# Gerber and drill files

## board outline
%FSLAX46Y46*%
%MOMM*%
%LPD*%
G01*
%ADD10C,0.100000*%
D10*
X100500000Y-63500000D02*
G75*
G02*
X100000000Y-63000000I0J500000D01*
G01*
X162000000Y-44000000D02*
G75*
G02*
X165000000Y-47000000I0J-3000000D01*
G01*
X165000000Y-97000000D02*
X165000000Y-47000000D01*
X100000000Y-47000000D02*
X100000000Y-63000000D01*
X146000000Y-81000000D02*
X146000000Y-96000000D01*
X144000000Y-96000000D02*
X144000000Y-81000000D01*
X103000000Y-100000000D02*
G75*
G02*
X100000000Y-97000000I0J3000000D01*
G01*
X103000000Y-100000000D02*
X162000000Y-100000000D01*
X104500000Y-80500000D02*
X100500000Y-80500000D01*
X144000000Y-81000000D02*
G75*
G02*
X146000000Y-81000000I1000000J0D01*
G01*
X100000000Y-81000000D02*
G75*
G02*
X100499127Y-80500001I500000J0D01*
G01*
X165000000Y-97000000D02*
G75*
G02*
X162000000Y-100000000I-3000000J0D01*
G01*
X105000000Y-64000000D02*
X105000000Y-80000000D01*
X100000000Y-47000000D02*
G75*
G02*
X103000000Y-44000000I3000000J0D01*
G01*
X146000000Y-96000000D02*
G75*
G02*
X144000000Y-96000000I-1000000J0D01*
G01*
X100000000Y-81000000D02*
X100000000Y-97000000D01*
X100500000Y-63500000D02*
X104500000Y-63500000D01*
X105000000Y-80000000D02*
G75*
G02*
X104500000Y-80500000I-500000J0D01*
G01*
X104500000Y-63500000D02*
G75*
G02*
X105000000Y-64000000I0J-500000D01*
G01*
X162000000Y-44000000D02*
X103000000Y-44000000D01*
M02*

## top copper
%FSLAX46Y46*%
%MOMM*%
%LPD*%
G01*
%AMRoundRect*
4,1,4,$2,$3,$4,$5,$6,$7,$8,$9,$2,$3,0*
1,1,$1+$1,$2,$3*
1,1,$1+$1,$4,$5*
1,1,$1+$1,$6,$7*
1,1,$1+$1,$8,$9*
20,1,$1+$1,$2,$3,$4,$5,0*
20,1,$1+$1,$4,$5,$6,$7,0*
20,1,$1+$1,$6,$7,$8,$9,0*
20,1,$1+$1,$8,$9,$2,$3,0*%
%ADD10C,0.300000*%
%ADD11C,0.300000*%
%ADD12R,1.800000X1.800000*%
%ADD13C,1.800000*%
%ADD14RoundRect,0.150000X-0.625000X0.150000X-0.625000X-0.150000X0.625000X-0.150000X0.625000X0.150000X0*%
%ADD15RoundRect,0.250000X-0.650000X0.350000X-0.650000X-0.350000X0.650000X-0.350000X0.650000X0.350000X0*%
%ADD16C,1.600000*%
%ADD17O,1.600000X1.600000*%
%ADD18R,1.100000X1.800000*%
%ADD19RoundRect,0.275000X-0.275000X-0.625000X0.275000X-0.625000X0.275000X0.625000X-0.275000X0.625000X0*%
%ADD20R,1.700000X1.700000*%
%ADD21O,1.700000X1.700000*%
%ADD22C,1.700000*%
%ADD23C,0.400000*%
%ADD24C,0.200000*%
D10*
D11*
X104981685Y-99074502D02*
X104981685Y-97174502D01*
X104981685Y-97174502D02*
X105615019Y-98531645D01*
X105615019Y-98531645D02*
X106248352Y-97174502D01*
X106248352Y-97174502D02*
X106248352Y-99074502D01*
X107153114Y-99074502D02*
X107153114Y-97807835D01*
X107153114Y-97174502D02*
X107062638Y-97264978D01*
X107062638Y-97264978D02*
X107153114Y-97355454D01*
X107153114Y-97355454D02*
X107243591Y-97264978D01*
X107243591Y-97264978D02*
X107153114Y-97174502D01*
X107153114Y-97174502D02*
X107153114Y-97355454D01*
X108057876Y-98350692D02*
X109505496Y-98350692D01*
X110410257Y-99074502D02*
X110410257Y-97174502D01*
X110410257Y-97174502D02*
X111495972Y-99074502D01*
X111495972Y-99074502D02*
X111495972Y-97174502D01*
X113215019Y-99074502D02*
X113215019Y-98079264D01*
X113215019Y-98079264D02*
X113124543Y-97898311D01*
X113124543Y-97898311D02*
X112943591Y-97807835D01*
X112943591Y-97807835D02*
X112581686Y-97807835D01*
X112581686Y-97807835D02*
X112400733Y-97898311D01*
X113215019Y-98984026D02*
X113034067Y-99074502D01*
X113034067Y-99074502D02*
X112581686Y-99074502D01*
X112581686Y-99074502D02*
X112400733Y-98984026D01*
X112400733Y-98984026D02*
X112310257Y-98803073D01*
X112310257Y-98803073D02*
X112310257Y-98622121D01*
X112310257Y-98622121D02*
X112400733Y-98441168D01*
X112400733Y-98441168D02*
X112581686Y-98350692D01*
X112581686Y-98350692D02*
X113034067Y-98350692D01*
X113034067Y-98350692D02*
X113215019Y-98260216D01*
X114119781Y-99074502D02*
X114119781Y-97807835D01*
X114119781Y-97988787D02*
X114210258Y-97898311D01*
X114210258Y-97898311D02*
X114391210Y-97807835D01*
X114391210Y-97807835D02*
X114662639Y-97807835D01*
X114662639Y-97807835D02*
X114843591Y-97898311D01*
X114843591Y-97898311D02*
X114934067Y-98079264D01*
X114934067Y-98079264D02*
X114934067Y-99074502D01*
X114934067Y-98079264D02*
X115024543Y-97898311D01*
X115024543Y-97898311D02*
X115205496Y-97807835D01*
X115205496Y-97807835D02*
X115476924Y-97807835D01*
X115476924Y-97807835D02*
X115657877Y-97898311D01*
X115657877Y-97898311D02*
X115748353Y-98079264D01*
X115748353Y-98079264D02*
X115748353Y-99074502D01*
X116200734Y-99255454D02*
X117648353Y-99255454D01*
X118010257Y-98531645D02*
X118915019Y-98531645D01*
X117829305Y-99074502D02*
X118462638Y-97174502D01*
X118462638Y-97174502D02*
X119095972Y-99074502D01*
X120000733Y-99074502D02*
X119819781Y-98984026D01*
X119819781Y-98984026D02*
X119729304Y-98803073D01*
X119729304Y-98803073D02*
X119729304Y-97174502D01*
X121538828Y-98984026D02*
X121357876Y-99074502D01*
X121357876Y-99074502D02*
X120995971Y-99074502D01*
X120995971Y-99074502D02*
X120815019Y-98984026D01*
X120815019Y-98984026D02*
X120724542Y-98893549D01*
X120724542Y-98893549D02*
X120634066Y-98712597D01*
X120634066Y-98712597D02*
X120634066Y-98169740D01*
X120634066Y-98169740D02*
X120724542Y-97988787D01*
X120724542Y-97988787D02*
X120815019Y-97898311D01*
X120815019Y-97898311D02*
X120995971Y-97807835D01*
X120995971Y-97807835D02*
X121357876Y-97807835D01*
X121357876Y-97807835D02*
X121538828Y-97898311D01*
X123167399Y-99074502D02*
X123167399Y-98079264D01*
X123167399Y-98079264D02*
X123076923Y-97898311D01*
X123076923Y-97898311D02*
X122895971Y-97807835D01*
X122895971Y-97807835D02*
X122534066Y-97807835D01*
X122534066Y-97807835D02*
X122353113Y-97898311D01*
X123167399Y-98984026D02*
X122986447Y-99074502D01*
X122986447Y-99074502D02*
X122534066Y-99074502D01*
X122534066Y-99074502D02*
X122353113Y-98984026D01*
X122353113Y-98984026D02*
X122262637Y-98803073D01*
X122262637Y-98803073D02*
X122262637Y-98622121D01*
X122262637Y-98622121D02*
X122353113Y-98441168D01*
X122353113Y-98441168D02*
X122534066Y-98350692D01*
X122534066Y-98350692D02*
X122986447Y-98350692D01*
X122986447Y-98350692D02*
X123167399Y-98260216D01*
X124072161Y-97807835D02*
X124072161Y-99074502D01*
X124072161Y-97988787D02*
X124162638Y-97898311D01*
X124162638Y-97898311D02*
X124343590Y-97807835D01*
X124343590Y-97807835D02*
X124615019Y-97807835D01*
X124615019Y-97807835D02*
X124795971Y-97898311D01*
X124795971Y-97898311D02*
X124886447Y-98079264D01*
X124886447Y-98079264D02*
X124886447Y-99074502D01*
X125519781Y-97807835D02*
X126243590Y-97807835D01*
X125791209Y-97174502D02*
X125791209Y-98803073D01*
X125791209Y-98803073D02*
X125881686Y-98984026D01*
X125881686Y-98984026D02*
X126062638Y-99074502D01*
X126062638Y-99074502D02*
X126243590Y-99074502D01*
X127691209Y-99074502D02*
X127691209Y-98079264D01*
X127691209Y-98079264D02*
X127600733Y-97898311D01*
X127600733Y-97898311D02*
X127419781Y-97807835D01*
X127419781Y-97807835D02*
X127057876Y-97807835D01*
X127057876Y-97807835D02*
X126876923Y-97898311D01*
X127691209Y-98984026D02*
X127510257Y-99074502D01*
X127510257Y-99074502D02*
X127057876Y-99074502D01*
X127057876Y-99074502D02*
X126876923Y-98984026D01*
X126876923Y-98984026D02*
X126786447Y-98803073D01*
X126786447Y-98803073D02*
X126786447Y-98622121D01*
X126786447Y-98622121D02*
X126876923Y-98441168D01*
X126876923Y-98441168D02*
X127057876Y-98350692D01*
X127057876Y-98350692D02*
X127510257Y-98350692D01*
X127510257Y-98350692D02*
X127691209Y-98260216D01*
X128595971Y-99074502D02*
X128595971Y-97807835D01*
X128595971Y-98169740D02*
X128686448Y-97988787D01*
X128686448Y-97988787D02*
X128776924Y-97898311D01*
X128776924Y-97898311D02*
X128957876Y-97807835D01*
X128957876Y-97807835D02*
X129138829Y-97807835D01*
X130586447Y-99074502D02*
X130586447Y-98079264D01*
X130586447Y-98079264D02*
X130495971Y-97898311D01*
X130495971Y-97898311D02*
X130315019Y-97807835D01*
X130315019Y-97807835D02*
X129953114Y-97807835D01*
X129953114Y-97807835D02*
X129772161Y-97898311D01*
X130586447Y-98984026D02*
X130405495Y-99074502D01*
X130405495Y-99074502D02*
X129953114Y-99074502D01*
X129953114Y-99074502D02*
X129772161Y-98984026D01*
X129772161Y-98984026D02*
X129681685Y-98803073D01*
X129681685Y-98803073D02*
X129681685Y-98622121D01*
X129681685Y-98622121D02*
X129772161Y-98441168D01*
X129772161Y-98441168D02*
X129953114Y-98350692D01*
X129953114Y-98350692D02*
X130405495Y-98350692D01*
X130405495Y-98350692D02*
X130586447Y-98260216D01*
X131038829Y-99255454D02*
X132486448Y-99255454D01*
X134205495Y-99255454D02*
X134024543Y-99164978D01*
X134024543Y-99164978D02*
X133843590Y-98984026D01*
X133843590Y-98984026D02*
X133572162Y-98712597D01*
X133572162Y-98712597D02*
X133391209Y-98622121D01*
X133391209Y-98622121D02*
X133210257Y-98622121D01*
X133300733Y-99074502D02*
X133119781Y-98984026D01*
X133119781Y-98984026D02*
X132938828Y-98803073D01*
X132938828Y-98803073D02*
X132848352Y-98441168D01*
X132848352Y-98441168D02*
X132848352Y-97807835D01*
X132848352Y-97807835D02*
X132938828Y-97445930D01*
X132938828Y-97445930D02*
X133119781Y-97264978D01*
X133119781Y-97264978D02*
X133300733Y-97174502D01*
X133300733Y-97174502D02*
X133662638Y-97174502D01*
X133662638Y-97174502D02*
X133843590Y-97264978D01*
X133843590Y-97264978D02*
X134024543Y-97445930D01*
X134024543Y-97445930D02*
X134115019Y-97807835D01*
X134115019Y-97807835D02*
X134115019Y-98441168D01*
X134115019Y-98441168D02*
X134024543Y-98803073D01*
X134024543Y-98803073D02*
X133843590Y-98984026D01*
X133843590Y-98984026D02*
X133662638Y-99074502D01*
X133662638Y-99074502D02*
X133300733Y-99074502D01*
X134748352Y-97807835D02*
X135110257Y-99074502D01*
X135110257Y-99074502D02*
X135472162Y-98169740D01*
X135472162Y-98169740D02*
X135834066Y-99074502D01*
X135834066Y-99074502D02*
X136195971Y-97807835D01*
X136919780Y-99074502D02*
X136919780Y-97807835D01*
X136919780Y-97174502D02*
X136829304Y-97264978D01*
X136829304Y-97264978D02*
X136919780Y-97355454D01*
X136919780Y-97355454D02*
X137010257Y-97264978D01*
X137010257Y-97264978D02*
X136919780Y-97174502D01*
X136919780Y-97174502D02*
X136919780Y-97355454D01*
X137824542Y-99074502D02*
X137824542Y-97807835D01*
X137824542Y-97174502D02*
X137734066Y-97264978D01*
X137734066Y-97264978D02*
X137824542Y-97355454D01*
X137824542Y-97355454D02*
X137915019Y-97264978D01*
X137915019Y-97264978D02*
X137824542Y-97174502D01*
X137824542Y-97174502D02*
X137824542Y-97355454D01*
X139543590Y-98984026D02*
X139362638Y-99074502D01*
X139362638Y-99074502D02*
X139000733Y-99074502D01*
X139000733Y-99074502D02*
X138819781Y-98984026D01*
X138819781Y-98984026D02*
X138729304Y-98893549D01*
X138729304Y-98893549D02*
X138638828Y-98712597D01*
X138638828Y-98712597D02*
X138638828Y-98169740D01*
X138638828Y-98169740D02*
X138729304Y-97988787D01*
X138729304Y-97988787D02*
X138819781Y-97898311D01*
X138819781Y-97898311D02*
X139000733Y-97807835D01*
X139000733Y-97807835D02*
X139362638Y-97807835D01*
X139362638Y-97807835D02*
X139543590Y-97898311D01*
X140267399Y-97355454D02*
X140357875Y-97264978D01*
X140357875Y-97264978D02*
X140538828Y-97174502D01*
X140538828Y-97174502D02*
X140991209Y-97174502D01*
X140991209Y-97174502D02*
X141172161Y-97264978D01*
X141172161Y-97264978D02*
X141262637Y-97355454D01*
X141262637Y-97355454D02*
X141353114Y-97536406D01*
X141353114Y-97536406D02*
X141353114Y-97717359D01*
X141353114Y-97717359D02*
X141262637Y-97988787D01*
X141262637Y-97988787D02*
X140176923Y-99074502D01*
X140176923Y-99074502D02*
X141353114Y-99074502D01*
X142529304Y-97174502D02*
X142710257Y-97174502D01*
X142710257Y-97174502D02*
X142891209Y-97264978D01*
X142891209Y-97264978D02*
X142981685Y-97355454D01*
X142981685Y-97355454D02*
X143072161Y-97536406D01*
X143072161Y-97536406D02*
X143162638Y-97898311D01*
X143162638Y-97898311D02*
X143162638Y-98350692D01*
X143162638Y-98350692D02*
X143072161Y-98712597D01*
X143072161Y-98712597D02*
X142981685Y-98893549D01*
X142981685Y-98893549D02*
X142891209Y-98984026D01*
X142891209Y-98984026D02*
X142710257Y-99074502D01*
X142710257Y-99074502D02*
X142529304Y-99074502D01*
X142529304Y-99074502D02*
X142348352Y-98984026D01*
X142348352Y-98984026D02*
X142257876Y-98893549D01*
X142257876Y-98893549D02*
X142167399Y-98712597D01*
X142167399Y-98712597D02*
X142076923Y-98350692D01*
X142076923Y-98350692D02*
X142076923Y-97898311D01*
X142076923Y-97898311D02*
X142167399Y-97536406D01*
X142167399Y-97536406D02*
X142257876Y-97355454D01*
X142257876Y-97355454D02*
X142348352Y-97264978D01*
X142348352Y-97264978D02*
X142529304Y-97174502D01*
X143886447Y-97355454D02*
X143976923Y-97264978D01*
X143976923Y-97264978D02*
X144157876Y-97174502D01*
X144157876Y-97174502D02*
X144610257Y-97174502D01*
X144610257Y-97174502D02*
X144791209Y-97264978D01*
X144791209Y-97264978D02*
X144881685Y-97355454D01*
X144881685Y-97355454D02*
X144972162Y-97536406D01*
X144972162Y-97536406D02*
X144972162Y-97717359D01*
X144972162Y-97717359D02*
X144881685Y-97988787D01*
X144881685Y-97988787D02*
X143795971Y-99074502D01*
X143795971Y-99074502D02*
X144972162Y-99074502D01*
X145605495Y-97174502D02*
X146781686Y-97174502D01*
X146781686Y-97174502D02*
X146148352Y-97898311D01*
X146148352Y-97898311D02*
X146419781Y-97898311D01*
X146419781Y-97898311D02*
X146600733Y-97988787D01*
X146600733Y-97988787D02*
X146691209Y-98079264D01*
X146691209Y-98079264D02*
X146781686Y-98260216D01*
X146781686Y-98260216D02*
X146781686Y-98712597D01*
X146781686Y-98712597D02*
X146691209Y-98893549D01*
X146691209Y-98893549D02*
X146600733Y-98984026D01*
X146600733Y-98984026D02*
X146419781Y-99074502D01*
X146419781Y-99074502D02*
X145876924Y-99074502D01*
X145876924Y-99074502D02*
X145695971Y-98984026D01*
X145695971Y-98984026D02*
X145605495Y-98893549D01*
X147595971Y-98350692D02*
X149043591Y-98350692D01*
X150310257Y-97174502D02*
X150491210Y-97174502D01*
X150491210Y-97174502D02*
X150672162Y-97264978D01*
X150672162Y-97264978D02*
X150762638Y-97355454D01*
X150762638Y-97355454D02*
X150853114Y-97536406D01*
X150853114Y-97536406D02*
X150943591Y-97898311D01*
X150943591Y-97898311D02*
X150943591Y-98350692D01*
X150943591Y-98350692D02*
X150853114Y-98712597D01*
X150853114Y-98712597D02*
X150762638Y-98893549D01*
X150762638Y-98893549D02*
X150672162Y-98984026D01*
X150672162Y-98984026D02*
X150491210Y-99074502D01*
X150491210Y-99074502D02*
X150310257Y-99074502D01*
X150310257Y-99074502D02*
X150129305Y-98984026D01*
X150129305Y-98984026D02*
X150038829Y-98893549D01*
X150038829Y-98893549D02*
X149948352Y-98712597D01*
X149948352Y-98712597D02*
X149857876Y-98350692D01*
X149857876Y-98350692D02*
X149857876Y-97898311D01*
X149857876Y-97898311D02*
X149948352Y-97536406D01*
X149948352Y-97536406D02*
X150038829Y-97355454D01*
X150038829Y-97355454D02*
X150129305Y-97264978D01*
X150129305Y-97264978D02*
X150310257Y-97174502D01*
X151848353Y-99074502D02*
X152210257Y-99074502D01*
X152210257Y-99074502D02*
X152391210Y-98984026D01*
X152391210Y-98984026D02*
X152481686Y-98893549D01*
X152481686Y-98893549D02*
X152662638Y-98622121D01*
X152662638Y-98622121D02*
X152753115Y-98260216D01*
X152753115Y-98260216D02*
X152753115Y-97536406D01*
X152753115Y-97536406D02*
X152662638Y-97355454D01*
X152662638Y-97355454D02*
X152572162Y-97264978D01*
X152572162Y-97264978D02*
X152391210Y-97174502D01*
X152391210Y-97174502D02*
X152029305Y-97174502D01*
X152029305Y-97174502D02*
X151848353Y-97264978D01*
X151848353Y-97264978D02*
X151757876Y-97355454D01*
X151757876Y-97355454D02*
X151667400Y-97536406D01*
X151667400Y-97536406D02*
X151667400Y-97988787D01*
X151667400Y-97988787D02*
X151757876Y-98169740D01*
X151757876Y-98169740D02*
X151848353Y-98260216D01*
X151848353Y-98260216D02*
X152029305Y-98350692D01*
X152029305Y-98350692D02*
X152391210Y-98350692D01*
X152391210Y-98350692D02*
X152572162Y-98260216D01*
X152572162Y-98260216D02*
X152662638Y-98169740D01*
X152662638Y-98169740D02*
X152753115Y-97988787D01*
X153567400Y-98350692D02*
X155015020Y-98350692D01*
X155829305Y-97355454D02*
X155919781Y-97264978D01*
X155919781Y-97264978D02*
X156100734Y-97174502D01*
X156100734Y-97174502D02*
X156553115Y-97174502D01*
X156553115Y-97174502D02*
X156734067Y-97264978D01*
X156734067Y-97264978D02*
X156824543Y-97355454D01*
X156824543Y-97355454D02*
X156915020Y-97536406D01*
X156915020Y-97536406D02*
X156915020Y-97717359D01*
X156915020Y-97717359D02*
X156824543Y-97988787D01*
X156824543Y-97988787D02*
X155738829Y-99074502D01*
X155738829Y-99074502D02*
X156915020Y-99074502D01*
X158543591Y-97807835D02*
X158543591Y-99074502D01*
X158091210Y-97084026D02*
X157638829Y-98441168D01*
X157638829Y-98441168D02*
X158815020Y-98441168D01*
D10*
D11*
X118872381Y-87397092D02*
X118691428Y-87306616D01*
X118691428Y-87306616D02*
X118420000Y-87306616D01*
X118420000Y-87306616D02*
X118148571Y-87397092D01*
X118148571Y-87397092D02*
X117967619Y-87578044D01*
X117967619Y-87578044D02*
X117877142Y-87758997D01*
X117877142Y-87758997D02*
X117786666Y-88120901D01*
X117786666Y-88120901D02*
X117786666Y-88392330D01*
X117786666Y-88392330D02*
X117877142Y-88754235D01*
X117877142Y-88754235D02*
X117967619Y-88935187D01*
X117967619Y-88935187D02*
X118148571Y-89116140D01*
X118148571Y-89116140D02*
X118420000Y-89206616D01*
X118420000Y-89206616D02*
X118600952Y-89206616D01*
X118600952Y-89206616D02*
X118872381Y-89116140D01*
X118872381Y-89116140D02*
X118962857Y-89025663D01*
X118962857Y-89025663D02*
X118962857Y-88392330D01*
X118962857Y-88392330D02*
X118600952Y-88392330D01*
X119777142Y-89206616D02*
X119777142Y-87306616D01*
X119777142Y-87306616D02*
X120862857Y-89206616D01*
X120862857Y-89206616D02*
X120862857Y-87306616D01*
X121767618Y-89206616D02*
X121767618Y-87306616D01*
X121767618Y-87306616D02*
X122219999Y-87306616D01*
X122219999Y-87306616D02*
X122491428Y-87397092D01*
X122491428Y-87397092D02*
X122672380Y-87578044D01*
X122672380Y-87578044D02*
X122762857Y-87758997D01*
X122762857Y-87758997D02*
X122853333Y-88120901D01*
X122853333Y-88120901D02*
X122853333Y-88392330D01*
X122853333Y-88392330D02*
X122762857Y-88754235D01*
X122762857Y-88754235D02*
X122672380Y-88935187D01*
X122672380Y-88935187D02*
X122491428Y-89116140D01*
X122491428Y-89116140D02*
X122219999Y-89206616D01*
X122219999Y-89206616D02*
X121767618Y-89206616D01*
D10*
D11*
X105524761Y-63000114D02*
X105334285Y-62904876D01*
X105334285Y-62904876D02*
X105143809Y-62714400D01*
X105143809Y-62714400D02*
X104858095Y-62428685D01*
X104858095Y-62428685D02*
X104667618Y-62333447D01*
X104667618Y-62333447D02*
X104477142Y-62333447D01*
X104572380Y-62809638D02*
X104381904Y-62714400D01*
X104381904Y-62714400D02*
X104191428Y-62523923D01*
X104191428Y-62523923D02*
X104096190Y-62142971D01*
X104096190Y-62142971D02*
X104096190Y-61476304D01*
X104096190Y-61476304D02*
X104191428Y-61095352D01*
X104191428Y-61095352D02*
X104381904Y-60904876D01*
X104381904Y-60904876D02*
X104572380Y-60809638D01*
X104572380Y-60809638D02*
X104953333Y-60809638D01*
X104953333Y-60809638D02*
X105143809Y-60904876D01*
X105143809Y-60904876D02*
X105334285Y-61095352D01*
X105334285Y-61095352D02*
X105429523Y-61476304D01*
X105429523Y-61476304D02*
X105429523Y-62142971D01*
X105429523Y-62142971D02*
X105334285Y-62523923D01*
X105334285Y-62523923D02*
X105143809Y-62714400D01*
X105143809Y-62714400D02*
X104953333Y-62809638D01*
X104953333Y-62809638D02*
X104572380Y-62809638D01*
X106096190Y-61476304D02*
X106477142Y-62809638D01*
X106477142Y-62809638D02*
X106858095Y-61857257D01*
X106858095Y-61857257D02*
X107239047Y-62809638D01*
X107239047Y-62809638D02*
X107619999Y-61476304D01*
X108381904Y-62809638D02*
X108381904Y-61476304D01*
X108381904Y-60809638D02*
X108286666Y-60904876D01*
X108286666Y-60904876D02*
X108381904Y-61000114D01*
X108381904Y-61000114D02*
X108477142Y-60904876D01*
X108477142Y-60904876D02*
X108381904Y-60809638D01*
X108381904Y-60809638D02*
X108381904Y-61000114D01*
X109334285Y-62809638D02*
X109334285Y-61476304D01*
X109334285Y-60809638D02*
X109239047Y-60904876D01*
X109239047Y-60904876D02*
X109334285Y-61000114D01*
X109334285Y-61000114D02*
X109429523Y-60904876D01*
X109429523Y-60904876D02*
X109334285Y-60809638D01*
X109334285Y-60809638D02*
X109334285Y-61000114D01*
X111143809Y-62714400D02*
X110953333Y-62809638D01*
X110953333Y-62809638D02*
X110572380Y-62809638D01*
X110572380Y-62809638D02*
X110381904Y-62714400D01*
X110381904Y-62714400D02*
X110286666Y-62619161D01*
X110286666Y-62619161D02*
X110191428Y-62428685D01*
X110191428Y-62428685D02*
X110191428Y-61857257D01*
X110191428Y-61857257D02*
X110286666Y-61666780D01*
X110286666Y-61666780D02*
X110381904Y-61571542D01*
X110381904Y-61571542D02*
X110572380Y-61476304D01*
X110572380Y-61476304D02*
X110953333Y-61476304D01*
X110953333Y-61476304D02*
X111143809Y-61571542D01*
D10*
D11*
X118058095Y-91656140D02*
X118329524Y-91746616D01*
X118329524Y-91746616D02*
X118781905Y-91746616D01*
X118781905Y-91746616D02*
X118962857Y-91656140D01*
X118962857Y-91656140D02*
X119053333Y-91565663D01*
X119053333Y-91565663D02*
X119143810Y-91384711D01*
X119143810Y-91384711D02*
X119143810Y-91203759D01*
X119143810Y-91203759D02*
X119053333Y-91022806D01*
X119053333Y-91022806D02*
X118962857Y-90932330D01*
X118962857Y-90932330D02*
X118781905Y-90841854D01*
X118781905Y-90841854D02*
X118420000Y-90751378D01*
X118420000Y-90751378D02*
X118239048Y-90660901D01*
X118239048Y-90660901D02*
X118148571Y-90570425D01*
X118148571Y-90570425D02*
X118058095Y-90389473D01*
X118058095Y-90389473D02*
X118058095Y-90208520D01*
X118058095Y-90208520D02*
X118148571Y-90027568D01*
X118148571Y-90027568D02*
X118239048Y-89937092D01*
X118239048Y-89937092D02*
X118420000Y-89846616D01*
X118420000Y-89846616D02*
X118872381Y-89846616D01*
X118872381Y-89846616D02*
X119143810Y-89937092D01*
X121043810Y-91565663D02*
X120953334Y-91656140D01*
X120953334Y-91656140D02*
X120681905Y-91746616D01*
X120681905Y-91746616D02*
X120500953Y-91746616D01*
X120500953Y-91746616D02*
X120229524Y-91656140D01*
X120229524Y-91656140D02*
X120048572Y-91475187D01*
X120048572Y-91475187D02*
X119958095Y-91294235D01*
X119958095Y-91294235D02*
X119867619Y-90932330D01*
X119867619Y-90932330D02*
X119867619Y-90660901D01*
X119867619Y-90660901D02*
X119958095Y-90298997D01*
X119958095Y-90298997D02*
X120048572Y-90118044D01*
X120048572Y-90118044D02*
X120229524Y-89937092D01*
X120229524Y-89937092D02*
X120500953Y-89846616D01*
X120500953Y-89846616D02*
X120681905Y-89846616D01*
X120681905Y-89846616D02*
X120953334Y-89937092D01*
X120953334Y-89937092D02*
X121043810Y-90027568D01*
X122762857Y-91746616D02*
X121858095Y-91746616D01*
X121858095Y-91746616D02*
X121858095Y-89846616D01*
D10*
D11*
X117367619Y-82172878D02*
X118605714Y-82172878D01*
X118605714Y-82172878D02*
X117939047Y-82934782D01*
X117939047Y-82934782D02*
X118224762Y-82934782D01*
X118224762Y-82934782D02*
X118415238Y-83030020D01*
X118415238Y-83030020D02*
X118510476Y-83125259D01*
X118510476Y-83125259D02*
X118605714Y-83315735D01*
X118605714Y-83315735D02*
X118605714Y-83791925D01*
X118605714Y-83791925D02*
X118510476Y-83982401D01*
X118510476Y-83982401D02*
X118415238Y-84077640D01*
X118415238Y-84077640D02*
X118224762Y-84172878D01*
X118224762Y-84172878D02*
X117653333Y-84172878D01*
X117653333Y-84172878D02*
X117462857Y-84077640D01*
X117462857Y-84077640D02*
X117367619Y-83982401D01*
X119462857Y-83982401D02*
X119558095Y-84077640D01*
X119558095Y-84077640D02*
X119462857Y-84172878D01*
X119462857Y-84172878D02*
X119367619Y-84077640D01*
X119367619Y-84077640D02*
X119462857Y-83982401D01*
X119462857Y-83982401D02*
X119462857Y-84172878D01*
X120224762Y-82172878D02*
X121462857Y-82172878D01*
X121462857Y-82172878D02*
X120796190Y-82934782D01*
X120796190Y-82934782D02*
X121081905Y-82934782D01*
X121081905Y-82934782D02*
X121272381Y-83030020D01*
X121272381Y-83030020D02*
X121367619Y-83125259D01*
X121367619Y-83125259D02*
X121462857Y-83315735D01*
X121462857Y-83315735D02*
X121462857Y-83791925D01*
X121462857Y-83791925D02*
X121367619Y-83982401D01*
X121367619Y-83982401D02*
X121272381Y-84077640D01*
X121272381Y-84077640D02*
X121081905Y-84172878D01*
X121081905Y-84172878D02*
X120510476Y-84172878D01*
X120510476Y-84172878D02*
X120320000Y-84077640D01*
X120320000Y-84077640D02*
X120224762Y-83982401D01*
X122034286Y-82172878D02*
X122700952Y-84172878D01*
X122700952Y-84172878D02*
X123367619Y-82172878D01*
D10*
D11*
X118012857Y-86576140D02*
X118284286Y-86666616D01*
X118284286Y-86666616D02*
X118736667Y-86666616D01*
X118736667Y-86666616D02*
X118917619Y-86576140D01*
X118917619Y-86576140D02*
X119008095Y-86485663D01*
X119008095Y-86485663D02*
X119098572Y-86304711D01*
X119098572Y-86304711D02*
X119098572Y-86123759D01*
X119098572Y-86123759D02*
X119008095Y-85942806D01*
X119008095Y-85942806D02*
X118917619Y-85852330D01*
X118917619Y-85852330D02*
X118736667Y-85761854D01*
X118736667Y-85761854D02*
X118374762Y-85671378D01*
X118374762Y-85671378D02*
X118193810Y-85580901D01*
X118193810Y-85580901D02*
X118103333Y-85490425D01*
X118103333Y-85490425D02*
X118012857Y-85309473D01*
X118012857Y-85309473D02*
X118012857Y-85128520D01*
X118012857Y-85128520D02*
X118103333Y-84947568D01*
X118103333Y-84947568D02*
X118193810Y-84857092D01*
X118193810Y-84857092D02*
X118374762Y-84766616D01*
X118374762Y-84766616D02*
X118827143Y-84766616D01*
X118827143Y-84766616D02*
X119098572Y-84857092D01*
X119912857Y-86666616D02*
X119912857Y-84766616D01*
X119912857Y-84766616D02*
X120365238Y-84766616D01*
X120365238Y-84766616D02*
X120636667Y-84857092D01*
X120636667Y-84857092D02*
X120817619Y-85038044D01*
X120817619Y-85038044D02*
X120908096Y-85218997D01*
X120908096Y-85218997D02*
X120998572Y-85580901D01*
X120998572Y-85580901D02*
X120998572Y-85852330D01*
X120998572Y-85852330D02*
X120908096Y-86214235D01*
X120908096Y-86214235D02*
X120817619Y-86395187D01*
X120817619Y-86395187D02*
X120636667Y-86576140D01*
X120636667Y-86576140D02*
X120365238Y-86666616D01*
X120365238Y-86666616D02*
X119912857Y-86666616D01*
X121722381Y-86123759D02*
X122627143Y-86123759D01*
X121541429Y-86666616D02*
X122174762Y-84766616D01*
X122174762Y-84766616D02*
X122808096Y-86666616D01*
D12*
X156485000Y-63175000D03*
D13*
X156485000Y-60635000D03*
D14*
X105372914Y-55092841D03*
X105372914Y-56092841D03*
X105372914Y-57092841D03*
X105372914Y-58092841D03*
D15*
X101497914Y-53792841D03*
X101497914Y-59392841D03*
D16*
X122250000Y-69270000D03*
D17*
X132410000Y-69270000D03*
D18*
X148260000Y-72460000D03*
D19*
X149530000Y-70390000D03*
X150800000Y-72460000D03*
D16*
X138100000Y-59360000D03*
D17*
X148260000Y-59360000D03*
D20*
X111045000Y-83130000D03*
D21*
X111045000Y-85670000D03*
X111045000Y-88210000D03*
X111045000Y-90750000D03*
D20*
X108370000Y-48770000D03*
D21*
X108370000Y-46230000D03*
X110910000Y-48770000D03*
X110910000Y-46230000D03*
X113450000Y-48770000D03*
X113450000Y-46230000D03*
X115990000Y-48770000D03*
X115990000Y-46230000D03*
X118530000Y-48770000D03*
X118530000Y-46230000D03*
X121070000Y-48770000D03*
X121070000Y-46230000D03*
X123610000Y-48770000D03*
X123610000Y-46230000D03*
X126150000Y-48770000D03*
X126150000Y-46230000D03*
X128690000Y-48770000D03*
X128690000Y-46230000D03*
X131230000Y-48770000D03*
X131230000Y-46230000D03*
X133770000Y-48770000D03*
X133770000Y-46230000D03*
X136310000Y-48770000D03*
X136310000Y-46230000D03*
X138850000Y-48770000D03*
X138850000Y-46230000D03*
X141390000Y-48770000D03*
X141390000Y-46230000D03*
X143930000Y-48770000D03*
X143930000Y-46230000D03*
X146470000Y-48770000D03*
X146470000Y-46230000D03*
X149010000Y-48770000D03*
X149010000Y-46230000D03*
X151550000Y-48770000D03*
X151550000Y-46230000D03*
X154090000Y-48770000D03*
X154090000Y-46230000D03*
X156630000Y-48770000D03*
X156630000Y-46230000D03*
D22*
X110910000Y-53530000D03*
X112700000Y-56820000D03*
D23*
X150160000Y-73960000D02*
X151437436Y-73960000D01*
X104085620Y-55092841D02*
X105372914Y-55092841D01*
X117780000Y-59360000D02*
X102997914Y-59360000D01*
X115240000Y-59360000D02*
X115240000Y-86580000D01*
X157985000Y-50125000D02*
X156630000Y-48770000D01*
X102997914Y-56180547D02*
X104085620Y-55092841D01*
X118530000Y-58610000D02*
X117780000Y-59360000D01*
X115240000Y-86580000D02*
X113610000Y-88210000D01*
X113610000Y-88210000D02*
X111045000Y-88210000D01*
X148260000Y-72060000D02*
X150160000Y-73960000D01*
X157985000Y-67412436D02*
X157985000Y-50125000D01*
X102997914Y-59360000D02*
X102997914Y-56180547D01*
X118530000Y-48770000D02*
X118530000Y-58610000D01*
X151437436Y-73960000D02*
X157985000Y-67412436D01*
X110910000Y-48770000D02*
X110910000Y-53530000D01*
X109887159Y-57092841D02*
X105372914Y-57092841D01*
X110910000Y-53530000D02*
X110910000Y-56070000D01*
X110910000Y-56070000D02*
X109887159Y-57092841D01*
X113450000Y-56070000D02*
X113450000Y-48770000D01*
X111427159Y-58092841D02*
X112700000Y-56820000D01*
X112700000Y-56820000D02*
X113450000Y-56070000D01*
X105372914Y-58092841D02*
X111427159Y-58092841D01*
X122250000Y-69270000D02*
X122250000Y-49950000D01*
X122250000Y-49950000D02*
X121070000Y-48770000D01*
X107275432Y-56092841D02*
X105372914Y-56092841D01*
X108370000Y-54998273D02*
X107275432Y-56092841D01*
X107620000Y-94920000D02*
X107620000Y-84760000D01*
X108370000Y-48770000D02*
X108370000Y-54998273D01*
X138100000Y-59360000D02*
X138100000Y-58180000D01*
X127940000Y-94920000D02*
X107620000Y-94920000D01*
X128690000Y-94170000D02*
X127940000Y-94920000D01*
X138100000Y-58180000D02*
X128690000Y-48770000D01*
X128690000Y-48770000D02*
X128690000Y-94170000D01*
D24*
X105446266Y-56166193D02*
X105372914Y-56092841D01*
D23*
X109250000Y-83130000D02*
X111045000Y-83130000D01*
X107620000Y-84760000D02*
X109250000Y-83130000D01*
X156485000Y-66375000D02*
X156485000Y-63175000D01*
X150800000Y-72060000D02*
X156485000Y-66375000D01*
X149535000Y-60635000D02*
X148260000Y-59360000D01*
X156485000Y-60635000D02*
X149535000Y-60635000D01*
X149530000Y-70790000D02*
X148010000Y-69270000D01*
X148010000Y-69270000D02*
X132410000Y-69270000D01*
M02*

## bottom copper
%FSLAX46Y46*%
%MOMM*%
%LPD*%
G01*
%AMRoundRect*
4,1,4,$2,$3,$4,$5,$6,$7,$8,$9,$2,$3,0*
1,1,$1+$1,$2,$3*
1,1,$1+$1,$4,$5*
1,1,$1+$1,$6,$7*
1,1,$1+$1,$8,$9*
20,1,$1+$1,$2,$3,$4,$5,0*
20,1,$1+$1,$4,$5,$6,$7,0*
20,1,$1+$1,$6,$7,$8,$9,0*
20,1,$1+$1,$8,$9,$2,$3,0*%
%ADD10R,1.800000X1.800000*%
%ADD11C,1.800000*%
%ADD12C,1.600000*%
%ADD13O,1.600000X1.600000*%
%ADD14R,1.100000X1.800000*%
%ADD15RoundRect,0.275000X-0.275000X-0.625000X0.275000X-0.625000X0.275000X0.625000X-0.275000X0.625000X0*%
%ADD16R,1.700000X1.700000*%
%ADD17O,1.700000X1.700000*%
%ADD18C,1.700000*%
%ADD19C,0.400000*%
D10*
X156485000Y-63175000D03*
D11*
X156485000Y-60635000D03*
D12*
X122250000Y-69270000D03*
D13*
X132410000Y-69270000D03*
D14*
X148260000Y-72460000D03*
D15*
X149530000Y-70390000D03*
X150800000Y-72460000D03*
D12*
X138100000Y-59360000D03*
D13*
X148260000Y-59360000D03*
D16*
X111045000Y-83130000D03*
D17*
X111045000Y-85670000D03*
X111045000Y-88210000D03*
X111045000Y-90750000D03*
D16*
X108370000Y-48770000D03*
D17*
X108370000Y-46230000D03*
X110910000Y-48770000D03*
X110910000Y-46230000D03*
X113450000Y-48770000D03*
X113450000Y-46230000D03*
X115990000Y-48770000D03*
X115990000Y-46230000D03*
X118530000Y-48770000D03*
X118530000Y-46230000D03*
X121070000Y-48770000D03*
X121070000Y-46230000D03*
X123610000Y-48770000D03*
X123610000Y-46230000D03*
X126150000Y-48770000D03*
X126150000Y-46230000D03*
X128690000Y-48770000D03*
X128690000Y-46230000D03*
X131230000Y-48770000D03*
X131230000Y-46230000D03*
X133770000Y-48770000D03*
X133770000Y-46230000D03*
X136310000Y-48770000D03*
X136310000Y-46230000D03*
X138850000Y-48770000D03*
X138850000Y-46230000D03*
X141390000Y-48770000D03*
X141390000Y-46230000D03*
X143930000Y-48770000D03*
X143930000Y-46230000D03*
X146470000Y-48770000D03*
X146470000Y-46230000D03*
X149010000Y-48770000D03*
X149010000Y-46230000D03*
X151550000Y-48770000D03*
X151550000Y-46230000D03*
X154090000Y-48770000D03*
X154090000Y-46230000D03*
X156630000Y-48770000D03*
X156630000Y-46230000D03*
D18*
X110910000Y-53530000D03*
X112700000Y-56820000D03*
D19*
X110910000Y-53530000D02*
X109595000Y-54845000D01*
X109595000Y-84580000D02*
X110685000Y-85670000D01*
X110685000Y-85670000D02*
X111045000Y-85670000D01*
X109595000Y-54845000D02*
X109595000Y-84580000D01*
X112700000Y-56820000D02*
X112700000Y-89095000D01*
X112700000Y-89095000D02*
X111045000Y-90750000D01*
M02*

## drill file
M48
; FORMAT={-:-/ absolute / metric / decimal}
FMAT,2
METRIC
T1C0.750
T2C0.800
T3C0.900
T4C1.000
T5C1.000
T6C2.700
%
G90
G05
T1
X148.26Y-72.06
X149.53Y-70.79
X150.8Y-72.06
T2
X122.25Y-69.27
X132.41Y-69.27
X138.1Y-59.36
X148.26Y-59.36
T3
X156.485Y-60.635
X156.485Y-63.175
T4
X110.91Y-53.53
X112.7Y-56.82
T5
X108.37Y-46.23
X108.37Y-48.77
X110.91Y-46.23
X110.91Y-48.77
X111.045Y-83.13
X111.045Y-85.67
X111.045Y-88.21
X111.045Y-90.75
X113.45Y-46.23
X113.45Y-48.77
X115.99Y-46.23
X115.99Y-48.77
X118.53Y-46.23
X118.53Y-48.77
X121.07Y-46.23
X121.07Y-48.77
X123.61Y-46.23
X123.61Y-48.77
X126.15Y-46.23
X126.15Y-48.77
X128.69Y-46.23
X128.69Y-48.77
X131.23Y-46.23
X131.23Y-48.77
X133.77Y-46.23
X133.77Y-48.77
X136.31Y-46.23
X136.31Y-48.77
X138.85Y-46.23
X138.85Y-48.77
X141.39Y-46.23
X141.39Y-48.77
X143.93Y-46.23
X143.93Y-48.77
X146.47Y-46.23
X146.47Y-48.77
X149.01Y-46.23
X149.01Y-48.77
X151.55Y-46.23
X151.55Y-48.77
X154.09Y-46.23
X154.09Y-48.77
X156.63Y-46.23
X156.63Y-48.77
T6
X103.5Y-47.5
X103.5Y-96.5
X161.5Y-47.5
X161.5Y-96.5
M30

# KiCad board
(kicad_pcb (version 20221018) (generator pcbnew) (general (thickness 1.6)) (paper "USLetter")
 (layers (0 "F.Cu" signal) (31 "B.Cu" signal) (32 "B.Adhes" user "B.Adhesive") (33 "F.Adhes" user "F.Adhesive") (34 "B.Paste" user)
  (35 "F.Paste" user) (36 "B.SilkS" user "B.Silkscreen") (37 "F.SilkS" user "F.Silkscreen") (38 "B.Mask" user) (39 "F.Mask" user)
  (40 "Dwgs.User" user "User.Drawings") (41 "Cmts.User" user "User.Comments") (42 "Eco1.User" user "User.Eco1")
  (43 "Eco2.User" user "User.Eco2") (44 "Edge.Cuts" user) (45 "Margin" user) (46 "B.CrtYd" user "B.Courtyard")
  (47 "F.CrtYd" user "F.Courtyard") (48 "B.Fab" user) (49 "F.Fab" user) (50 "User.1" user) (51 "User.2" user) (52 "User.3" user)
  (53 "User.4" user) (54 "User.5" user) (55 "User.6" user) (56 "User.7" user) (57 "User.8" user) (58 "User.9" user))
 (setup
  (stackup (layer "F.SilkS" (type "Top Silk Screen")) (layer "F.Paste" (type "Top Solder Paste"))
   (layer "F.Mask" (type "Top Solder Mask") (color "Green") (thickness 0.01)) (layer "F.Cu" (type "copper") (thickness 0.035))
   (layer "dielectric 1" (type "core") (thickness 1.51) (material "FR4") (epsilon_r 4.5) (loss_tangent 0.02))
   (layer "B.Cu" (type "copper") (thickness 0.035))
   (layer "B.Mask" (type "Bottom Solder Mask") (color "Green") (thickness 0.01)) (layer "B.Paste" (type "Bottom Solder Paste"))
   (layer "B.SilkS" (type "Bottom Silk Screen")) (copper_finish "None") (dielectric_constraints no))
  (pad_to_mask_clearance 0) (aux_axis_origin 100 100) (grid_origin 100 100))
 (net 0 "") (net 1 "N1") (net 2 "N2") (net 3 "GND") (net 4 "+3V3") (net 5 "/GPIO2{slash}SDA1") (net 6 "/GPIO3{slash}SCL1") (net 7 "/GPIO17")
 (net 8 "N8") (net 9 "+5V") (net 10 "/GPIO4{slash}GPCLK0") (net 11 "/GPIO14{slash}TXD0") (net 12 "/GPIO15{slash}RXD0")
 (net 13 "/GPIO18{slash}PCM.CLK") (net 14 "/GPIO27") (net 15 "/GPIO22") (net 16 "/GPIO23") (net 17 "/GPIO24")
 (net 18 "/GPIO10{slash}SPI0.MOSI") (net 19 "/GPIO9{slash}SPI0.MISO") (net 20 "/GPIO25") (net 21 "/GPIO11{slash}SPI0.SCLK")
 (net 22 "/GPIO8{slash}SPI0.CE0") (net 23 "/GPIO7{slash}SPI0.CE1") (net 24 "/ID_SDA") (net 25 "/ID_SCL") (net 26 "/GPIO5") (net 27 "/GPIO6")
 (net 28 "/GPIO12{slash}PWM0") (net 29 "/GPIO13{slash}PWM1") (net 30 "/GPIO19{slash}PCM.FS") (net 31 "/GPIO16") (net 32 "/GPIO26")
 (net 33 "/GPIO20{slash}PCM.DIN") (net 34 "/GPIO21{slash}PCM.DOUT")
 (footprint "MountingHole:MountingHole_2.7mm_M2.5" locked (layer "F.Cu") (at 161.5 47.5)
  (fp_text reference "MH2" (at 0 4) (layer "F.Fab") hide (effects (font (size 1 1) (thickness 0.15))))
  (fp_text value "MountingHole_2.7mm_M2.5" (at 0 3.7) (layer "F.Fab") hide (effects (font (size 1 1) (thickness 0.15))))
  (pad "" np_thru_hole circle locked (at 0 0) (size 2.7 2.7) (drill 2.7) (layers "*.Cu" "*.Mask")))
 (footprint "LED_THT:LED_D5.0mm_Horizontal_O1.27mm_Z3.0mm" (layer "F.Cu") (at 156.485 63.175 90)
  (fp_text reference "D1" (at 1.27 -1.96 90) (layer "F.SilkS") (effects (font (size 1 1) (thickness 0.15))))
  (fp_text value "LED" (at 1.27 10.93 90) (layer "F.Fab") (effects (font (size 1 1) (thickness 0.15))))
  (pad "1" thru_hole rect (at 0 0 90) (size 1.8 1.8) (drill 0.9) (layers "*.Cu" "*.Mask") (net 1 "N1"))
  (pad "2" thru_hole circle (at 2.54 0 90) (size 1.8 1.8) (drill 0.9) (layers "*.Cu" "*.Mask") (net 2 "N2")))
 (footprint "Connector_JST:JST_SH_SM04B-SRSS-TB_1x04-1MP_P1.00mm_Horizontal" (layer "F.Cu") (at 103.372914 56.592841 -90)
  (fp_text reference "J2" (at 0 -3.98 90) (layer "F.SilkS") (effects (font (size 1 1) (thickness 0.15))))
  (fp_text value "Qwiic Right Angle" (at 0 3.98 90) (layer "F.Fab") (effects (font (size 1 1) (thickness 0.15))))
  (pad "1" smd roundrect (at -1.5 -2 270) (size 0.6 1.55) (layers "F.Cu" "F.Paste" "F.Mask") (roundrect_rratio 0.25) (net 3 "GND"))
  (pad "2" smd roundrect (at -0.5 -2 270) (size 0.6 1.55) (layers "F.Cu" "F.Paste" "F.Mask") (roundrect_rratio 0.25) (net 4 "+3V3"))
  (pad "3" smd roundrect (at 0.5 -2 270) (size 0.6 1.55) (layers "F.Cu" "F.Paste" "F.Mask") (roundrect_rratio 0.25)
   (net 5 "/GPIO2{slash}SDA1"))
  (pad "4" smd roundrect (at 1.5 -2 270) (size 0.6 1.55) (layers "F.Cu" "F.Paste" "F.Mask") (roundrect_rratio 0.25)
   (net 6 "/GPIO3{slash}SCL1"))
  (pad "MP" smd roundrect (at -2.8 1.875 270) (size 1.2 1.8) (layers "F.Cu" "F.Paste" "F.Mask") (roundrect_rratio 0.2083333333))
  (pad "MP" smd roundrect (at 2.8 1.875 270) (size 1.2 1.8) (layers "F.Cu" "F.Paste" "F.Mask") (roundrect_rratio 0.2083333333)))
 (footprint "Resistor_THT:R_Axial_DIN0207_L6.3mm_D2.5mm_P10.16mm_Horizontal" (layer "F.Cu") (at 122.25 69.27)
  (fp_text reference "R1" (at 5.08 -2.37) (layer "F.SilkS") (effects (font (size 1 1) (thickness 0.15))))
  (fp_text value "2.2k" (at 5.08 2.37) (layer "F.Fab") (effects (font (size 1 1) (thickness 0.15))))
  (pad "1" thru_hole circle (at 0 0) (size 1.6 1.6) (drill 0.8) (layers "*.Cu" "*.Mask") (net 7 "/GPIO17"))
  (pad "2" thru_hole oval (at 10.16 0) (size 1.6 1.6) (drill 0.8) (layers "*.Cu" "*.Mask") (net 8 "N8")))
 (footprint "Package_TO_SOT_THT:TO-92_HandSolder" (layer "F.Cu") (at 148.26 72.06)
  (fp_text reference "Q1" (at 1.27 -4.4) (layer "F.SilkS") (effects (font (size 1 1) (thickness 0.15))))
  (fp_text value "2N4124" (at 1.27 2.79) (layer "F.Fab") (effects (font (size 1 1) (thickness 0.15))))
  (pad "1" thru_hole rect (at 0 0) (size 1.1 1.8) (drill 0.75 (offset 0 0.4)) (layers "*.Cu" "*.Mask") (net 3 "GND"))
  (pad "2" thru_hole roundrect (at 1.27 -1.27) (size 1.1 1.8) (drill 0.75 (offset 0 -0.4)) (layers "*.Cu" "*.Mask") (roundrect_rratio 0.25)
   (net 8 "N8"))
  (pad "3" thru_hole roundrect (at 2.54 0) (size 1.1 1.8) (drill 0.75 (offset 0 0.4)) (layers "*.Cu" "*.Mask") (roundrect_rratio 0.25)
   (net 1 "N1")))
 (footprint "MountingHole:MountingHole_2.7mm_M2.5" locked (layer "F.Cu") (at 103.5 96.5)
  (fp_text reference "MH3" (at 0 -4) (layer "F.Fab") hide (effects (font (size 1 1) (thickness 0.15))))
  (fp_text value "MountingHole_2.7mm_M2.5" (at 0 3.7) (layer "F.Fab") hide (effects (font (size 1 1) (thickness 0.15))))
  (pad "" np_thru_hole circle locked (at 0 0) (size 2.7 2.7) (drill 2.7) (layers "*.Cu" "*.Mask")))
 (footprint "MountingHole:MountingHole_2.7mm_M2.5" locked (layer "F.Cu") (at 103.5 47.5)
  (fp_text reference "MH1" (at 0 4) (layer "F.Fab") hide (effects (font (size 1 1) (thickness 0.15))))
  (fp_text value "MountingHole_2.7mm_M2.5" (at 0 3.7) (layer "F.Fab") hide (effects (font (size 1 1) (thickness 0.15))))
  (pad "" np_thru_hole circle locked (at 0 0) (size 2.7 2.7) (drill 2.7) (layers "*.Cu" "*.Mask")))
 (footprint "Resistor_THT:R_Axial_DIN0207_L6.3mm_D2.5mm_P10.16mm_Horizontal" (layer "F.Cu") (at 138.1 59.36)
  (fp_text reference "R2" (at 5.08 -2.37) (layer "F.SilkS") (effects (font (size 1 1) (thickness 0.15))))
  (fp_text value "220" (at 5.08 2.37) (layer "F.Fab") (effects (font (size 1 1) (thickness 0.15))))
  (pad "1" thru_hole circle (at 0 0) (size 1.6 1.6) (drill 0.8) (layers "*.Cu" "*.Mask") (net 4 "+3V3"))
  (pad "2" thru_hole oval (at 10.16 0) (size 1.6 1.6) (drill 0.8) (layers "*.Cu" "*.Mask") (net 2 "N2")))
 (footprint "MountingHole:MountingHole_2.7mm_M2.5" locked (layer "F.Cu") (at 161.5 96.5)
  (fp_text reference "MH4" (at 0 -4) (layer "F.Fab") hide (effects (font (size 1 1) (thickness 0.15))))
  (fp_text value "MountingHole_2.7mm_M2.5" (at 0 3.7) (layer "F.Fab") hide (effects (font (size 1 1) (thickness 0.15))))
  (pad "" np_thru_hole circle locked (at 0 0) (size 2.7 2.7) (drill 2.7) (layers "*.Cu" "*.Mask")))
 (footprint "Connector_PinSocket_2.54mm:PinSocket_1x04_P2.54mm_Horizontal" (layer "F.Cu") (at 111.045 83.13)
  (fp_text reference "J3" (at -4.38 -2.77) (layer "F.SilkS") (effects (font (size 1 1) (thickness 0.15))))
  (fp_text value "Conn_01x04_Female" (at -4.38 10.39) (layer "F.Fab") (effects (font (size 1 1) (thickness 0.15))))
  (pad "1" thru_hole rect (at 0 0) (size 1.7 1.7) (drill 1) (layers "*.Cu" "*.Mask") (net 4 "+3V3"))
  (pad "2" thru_hole oval (at 0 2.54) (size 1.7 1.7) (drill 1) (layers "*.Cu" "*.Mask") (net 5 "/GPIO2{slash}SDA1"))
  (pad "3" thru_hole oval (at 0 5.08) (size 1.7 1.7) (drill 1) (layers "*.Cu" "*.Mask") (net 3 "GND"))
  (pad "4" thru_hole oval (at 0 7.62) (size 1.7 1.7) (drill 1) (layers "*.Cu" "*.Mask") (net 6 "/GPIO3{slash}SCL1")))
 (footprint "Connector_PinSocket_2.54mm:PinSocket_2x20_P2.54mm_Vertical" (layer "B.Cu") (at 108.37 48.77 -90)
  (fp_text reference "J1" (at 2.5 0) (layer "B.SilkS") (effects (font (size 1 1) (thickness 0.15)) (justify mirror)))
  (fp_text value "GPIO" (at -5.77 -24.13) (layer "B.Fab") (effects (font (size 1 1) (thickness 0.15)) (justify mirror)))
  (pad "1" thru_hole rect (at 0 0 270) (size 1.7 1.7) (drill 1) (layers "*.Cu" "*.Mask") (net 4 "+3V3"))
  (pad "2" thru_hole oval (at -2.54 0 270) (size 1.7 1.7) (drill 1) (layers "*.Cu" "*.Mask") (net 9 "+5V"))
  (pad "3" thru_hole oval (at 0 -2.54 270) (size 1.7 1.7) (drill 1) (layers "*.Cu" "*.Mask") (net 5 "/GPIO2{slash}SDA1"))
  (pad "4" thru_hole oval (at -2.54 -2.54 270) (size 1.7 1.7) (drill 1) (layers "*.Cu" "*.Mask") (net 9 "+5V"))
  (pad "5" thru_hole oval (at 0 -5.08 270) (size 1.7 1.7) (drill 1) (layers "*.Cu" "*.Mask") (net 6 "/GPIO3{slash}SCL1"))
  (pad "6" thru_hole oval (at -2.54 -5.08 270) (size 1.7 1.7) (drill 1) (layers "*.Cu" "*.Mask") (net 3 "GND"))
  (pad "7" thru_hole oval (at 0 -7.62 270) (size 1.7 1.7) (drill 1) (layers "*.Cu" "*.Mask") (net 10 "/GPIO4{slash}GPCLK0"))
  (pad "8" thru_hole oval (at -2.54 -7.62 270) (size 1.7 1.7) (drill 1) (layers "*.Cu" "*.Mask") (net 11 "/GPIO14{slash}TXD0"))
  (pad "9" thru_hole oval (at 0 -10.16 270) (size 1.7 1.7) (drill 1) (layers "*.Cu" "*.Mask") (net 3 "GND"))
  (pad "10" thru_hole oval (at -2.54 -10.16 270) (size 1.7 1.7) (drill 1) (layers "*.Cu" "*.Mask") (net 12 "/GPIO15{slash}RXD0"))
  (pad "11" thru_hole oval (at 0 -12.7 270) (size 1.7 1.7) (drill 1) (layers "*.Cu" "*.Mask") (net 7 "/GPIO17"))
  (pad "12" thru_hole oval (at -2.54 -12.7 270) (size 1.7 1.7) (drill 1) (layers "*.Cu" "*.Mask") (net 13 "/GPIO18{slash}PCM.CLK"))
  (pad "13" thru_hole oval (at 0 -15.24 270) (size 1.7 1.7) (drill 1) (layers "*.Cu" "*.Mask") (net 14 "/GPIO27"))
  (pad "14" thru_hole oval (at -2.54 -15.24 270) (size 1.7 1.7) (drill 1) (layers "*.Cu" "*.Mask") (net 3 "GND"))
  (pad "15" thru_hole oval (at 0 -17.78 270) (size 1.7 1.7) (drill 1) (layers "*.Cu" "*.Mask") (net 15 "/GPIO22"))
  (pad "16" thru_hole oval (at -2.54 -17.78 270) (size 1.7 1.7) (drill 1) (layers "*.Cu" "*.Mask") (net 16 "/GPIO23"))
  (pad "17" thru_hole oval (at 0 -20.32 270) (size 1.7 1.7) (drill 1) (layers "*.Cu" "*.Mask") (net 4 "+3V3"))
  (pad "18" thru_hole oval (at -2.54 -20.32 270) (size 1.7 1.7) (drill 1) (layers "*.Cu" "*.Mask") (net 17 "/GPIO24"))
  (pad "19" thru_hole oval (at 0 -22.86 270) (size 1.7 1.7) (drill 1) (layers "*.Cu" "*.Mask") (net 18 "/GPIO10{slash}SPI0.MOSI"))
  (pad "20" thru_hole oval (at -2.54 -22.86 270) (size 1.7 1.7) (drill 1) (layers "*.Cu" "*.Mask") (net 3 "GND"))
  (pad "21" thru_hole oval (at 0 -25.4 270) (size 1.7 1.7) (drill 1) (layers "*.Cu" "*.Mask") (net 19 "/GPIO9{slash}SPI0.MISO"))
  (pad "22" thru_hole oval (at -2.54 -25.4 270) (size 1.7 1.7) (drill 1) (layers "*.Cu" "*.Mask") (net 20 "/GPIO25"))
  (pad "23" thru_hole oval (at 0 -27.94 270) (size 1.7 1.7) (drill 1) (layers "*.Cu" "*.Mask") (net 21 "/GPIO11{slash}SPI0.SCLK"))
  (pad "24" thru_hole oval (at -2.54 -27.94 270) (size 1.7 1.7) (drill 1) (layers "*.Cu" "*.Mask") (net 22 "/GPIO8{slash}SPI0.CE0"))
  (pad "25" thru_hole oval (at 0 -30.48 270) (size 1.7 1.7) (drill 1) (layers "*.Cu" "*.Mask") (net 3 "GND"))
  (pad "26" thru_hole oval (at -2.54 -30.48 270) (size 1.7 1.7) (drill 1) (layers "*.Cu" "*.Mask") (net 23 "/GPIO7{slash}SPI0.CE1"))
  (pad "27" thru_hole oval (at 0 -33.02 270) (size 1.7 1.7) (drill 1) (layers "*.Cu" "*.Mask") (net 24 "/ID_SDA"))
  (pad "28" thru_hole oval (at -2.54 -33.02 270) (size 1.7 1.7) (drill 1) (layers "*.Cu" "*.Mask") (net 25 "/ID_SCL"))
  (pad "29" thru_hole oval (at 0 -35.56 270) (size 1.7 1.7) (drill 1) (layers "*.Cu" "*.Mask") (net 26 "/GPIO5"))
  (pad "30" thru_hole oval (at -2.54 -35.56 270) (size 1.7 1.7) (drill 1) (layers "*.Cu" "*.Mask") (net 3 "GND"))
  (pad "31" thru_hole oval (at 0 -38.1 270) (size 1.7 1.7) (drill 1) (layers "*.Cu" "*.Mask") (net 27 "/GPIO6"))
  (pad "32" thru_hole oval (at -2.54 -38.1 270) (size 1.7 1.7) (drill 1) (layers "*.Cu" "*.Mask") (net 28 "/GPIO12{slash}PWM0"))
  (pad "33" thru_hole oval (at 0 -40.64 270) (size 1.7 1.7) (drill 1) (layers "*.Cu" "*.Mask") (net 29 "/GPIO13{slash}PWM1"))
  (pad "34" thru_hole oval (at -2.54 -40.64 270) (size 1.7 1.7) (drill 1) (layers "*.Cu" "*.Mask") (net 3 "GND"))
  (pad "35" thru_hole oval (at 0 -43.18 270) (size 1.7 1.7) (drill 1) (layers "*.Cu" "*.Mask") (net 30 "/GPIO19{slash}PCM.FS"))
  (pad "36" thru_hole oval (at -2.54 -43.18 270) (size 1.7 1.7) (drill 1) (layers "*.Cu" "*.Mask") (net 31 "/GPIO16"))
  (pad "37" thru_hole oval (at 0 -45.72 270) (size 1.7 1.7) (drill 1) (layers "*.Cu" "*.Mask") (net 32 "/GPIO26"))
  (pad "38" thru_hole oval (at -2.54 -45.72 270) (size 1.7 1.7) (drill 1) (layers "*.Cu" "*.Mask") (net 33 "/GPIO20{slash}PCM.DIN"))
  (pad "39" thru_hole oval (at 0 -48.26 270) (size 1.7 1.7) (drill 1) (layers "*.Cu" "*.Mask") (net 3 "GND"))
  (pad "40" thru_hole oval (at -2.54 -48.26 270) (size 1.7 1.7) (drill 1) (layers "*.Cu" "*.Mask") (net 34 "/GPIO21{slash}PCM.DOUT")))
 (gr_arc (start 100.5 63.5) (mid 100.146447 63.353553) (end 100 63) (stroke (width 0.1) (type solid)) (layer "Edge.Cuts"))
 (gr_arc (start 162 44) (mid 164.12132 44.87868) (end 165 47) (stroke (width 0.1) (type solid)) (layer "Edge.Cuts"))
 (gr_line (start 165 97) (end 165 47) (stroke (width 0.1) (type solid)) (layer "Edge.Cuts"))
 (gr_line (start 100 47) (end 100 63) (stroke (width 0.1) (type solid)) (layer "Edge.Cuts"))
 (gr_line (start 146 81) (end 146 96) (stroke (width 0.1) (type solid)) (layer "Edge.Cuts"))
 (gr_line (start 144 96) (end 144 81) (stroke (width 0.1) (type solid)) (layer "Edge.Cuts"))
 (gr_arc (start 103 100) (mid 100.87868 99.12132) (end 100 97) (stroke (width 0.1) (type solid)) (layer "Edge.Cuts"))
 (gr_line (start 103 100) (end 162 100) (stroke (width 0.1) (type solid)) (layer "Edge.Cuts"))
 (gr_line (start 104.5 80.5) (end 100.5 80.5) (stroke (width 0.1) (type solid)) (layer "Edge.Cuts"))
 (gr_arc (start 144 81) (mid 145 80) (end 146 81) (stroke (width 0.1) (type solid)) (layer "Edge.Cuts"))
 (gr_arc (start 100 81) (mid 100.146138 80.646755) (end 100.499127 80.500001) (stroke (width 0.1) (type solid)) (layer "Edge.Cuts"))
 (gr_arc (start 165 97) (mid 164.12132 99.12132) (end 162 100) (stroke (width 0.1) (type solid)) (layer "Edge.Cuts"))
 (gr_line (start 105 64) (end 105 80) (stroke (width 0.1) (type solid)) (layer "Edge.Cuts"))
 (gr_arc (start 100 47) (mid 100.87868 44.87868) (end 103 44) (stroke (width 0.1) (type solid)) (layer "Edge.Cuts"))
 (gr_arc (start 146 96) (mid 145 97) (end 144 96) (stroke (width 0.1) (type solid)) (layer "Edge.Cuts"))
 (gr_line (start 100 81) (end 100 97) (stroke (width 0.1) (type solid)) (layer "Edge.Cuts"))
 (gr_line (start 100.5 63.5) (end 104.5 63.5) (stroke (width 0.1) (type solid)) (layer "Edge.Cuts"))
 (gr_arc (start 105 80) (mid 104.853553 80.353553) (end 104.5 80.5) (stroke (width 0.1) (type solid)) (layer "Edge.Cuts"))
 (gr_arc (start 104.5 63.5) (mid 104.853553 63.646447) (end 105 64) (stroke (width 0.1) (type solid)) (layer "Edge.Cuts"))
 (gr_line (start 162 44) (end 103 44) (stroke (width 0.1) (type solid)) (layer "Edge.Cuts"))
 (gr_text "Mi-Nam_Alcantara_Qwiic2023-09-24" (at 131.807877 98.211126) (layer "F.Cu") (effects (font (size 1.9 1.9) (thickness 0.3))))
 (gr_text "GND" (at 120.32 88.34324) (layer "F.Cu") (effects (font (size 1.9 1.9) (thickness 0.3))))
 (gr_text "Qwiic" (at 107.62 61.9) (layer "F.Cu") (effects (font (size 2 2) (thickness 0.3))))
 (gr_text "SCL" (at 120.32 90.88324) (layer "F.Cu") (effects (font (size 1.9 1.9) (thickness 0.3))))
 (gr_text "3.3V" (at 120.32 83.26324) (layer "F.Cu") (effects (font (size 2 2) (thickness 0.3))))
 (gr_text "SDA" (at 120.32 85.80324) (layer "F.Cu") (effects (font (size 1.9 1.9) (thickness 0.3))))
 (segment (start 150.16 73.96) (end 151.437436 73.96) (width 0.4) (layer "F.Cu") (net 3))
 (segment (start 104.08562 55.092841) (end 105.372914 55.092841) (width 0.4) (layer "F.Cu") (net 3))
 (segment (start 117.78 59.36) (end 102.997914 59.36) (width 0.4) (layer "F.Cu") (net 3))
 (segment (start 115.24 59.36) (end 115.24 86.58) (width 0.4) (layer "F.Cu") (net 3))
 (segment (start 157.985 50.125) (end 156.63 48.77) (width 0.4) (layer "F.Cu") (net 3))
 (segment (start 102.997914 56.180547) (end 104.08562 55.092841) (width 0.4) (layer "F.Cu") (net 3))
 (segment (start 118.53 58.61) (end 117.78 59.36) (width 0.4) (layer "F.Cu") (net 3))
 (segment (start 115.24 86.58) (end 113.61 88.21) (width 0.4) (layer "F.Cu") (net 3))
 (segment (start 113.61 88.21) (end 111.045 88.21) (width 0.4) (layer "F.Cu") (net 3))
 (segment (start 148.26 72.06) (end 150.16 73.96) (width 0.4) (layer "F.Cu") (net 3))
 (segment (start 157.985 67.412436) (end 157.985 50.125) (width 0.4) (layer "F.Cu") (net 3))
 (segment (start 102.997914 59.36) (end 102.997914 56.180547) (width 0.4) (layer "F.Cu") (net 3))
 (segment (start 118.53 48.77) (end 118.53 58.61) (width 0.4) (layer "F.Cu") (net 3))
 (segment (start 151.437436 73.96) (end 157.985 67.412436) (width 0.4) (layer "F.Cu") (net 3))
 (segment (start 110.91 48.77) (end 110.91 53.53) (width 0.4) (layer "F.Cu") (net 5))
 (segment (start 109.887159 57.092841) (end 105.372914 57.092841) (width 0.4) (layer "F.Cu") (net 5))
 (segment (start 110.91 53.53) (end 110.91 56.07) (width 0.4) (layer "F.Cu") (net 5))
 (segment (start 110.91 56.07) (end 109.887159 57.092841) (width 0.4) (layer "F.Cu") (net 5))
 (via (at 110.91 53.53) (size 1.7) (drill 1) (layers "F.Cu" "B.Cu") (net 5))
 (segment (start 110.91 53.53) (end 109.595 54.845) (width 0.4) (layer "B.Cu") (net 5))
 (segment (start 109.595 84.58) (end 110.685 85.67) (width 0.4) (layer "B.Cu") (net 5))
 (segment (start 110.685 85.67) (end 111.045 85.67) (width 0.4) (layer "B.Cu") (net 5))
 (segment (start 109.595 54.845) (end 109.595 84.58) (width 0.4) (layer "B.Cu") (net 5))
 (segment (start 113.45 56.07) (end 113.45 48.77) (width 0.4) (layer "F.Cu") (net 6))
 (segment (start 111.427159 58.092841) (end 112.7 56.82) (width 0.4) (layer "F.Cu") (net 6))
 (segment (start 112.7 56.82) (end 113.45 56.07) (width 0.4) (layer "F.Cu") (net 6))
 (segment (start 105.372914 58.092841) (end 111.427159 58.092841) (width 0.4) (layer "F.Cu") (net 6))
 (via (at 112.7 56.82) (size 1.7) (drill 1) (layers "F.Cu" "B.Cu") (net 6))
 (segment (start 112.7 56.82) (end 112.7 89.095) (width 0.4) (layer "B.Cu") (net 6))
 (segment (start 112.7 89.095) (end 111.045 90.75) (width 0.4) (layer "B.Cu") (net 6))
 (segment (start 122.25 69.27) (end 122.25 49.95) (width 0.4) (layer "F.Cu") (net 7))
 (segment (start 122.25 49.95) (end 121.07 48.77) (width 0.4) (layer "F.Cu") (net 7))
 (segment (start 107.275432 56.092841) (end 105.372914 56.092841) (width 0.4) (layer "F.Cu") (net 4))
 (segment (start 108.37 54.998273) (end 107.275432 56.092841) (width 0.4) (layer "F.Cu") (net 4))
 (segment (start 107.62 94.92) (end 107.62 84.76) (width 0.4) (layer "F.Cu") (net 4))
 (segment (start 108.37 48.77) (end 108.37 54.998273) (width 0.4) (layer "F.Cu") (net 4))
 (segment (start 138.1 59.36) (end 138.1 58.18) (width 0.4) (layer "F.Cu") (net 4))
 (segment (start 127.94 94.92) (end 107.62 94.92) (width 0.4) (layer "F.Cu") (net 4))
 (segment (start 128.69 94.17) (end 127.94 94.92) (width 0.4) (layer "F.Cu") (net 4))
 (segment (start 138.1 58.18) (end 128.69 48.77) (width 0.4) (layer "F.Cu") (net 4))
 (segment (start 128.69 48.77) (end 128.69 94.17) (width 0.4) (layer "F.Cu") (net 4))
 (segment (start 105.446266 56.166193) (end 105.372914 56.092841) (width 0.2) (layer "F.Cu") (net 4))
 (segment (start 109.25 83.13) (end 111.045 83.13) (width 0.4) (layer "F.Cu") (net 4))
 (segment (start 107.62 84.76) (end 109.25 83.13) (width 0.4) (layer "F.Cu") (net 4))
 (segment (start 156.485 66.375) (end 156.485 63.175) (width 0.4) (layer "F.Cu") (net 1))
 (segment (start 150.8 72.06) (end 156.485 66.375) (width 0.4) (layer "F.Cu") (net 1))
 (segment (start 149.535 60.635) (end 148.26 59.36) (width 0.4) (layer "F.Cu") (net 2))
 (segment (start 156.485 60.635) (end 149.535 60.635) (width 0.4) (layer "F.Cu") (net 2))
 (segment (start 149.53 70.79) (end 148.01 69.27) (width 0.4) (layer "F.Cu") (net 8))
 (segment (start 148.01 69.27) (end 132.41 69.27) (width 0.4) (layer "F.Cu") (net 8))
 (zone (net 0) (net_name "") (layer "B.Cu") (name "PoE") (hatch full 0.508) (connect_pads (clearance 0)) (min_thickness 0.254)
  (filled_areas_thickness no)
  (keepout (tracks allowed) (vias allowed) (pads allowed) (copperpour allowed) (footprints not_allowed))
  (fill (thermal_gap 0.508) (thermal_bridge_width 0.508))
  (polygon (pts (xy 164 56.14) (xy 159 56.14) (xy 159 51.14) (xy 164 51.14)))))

